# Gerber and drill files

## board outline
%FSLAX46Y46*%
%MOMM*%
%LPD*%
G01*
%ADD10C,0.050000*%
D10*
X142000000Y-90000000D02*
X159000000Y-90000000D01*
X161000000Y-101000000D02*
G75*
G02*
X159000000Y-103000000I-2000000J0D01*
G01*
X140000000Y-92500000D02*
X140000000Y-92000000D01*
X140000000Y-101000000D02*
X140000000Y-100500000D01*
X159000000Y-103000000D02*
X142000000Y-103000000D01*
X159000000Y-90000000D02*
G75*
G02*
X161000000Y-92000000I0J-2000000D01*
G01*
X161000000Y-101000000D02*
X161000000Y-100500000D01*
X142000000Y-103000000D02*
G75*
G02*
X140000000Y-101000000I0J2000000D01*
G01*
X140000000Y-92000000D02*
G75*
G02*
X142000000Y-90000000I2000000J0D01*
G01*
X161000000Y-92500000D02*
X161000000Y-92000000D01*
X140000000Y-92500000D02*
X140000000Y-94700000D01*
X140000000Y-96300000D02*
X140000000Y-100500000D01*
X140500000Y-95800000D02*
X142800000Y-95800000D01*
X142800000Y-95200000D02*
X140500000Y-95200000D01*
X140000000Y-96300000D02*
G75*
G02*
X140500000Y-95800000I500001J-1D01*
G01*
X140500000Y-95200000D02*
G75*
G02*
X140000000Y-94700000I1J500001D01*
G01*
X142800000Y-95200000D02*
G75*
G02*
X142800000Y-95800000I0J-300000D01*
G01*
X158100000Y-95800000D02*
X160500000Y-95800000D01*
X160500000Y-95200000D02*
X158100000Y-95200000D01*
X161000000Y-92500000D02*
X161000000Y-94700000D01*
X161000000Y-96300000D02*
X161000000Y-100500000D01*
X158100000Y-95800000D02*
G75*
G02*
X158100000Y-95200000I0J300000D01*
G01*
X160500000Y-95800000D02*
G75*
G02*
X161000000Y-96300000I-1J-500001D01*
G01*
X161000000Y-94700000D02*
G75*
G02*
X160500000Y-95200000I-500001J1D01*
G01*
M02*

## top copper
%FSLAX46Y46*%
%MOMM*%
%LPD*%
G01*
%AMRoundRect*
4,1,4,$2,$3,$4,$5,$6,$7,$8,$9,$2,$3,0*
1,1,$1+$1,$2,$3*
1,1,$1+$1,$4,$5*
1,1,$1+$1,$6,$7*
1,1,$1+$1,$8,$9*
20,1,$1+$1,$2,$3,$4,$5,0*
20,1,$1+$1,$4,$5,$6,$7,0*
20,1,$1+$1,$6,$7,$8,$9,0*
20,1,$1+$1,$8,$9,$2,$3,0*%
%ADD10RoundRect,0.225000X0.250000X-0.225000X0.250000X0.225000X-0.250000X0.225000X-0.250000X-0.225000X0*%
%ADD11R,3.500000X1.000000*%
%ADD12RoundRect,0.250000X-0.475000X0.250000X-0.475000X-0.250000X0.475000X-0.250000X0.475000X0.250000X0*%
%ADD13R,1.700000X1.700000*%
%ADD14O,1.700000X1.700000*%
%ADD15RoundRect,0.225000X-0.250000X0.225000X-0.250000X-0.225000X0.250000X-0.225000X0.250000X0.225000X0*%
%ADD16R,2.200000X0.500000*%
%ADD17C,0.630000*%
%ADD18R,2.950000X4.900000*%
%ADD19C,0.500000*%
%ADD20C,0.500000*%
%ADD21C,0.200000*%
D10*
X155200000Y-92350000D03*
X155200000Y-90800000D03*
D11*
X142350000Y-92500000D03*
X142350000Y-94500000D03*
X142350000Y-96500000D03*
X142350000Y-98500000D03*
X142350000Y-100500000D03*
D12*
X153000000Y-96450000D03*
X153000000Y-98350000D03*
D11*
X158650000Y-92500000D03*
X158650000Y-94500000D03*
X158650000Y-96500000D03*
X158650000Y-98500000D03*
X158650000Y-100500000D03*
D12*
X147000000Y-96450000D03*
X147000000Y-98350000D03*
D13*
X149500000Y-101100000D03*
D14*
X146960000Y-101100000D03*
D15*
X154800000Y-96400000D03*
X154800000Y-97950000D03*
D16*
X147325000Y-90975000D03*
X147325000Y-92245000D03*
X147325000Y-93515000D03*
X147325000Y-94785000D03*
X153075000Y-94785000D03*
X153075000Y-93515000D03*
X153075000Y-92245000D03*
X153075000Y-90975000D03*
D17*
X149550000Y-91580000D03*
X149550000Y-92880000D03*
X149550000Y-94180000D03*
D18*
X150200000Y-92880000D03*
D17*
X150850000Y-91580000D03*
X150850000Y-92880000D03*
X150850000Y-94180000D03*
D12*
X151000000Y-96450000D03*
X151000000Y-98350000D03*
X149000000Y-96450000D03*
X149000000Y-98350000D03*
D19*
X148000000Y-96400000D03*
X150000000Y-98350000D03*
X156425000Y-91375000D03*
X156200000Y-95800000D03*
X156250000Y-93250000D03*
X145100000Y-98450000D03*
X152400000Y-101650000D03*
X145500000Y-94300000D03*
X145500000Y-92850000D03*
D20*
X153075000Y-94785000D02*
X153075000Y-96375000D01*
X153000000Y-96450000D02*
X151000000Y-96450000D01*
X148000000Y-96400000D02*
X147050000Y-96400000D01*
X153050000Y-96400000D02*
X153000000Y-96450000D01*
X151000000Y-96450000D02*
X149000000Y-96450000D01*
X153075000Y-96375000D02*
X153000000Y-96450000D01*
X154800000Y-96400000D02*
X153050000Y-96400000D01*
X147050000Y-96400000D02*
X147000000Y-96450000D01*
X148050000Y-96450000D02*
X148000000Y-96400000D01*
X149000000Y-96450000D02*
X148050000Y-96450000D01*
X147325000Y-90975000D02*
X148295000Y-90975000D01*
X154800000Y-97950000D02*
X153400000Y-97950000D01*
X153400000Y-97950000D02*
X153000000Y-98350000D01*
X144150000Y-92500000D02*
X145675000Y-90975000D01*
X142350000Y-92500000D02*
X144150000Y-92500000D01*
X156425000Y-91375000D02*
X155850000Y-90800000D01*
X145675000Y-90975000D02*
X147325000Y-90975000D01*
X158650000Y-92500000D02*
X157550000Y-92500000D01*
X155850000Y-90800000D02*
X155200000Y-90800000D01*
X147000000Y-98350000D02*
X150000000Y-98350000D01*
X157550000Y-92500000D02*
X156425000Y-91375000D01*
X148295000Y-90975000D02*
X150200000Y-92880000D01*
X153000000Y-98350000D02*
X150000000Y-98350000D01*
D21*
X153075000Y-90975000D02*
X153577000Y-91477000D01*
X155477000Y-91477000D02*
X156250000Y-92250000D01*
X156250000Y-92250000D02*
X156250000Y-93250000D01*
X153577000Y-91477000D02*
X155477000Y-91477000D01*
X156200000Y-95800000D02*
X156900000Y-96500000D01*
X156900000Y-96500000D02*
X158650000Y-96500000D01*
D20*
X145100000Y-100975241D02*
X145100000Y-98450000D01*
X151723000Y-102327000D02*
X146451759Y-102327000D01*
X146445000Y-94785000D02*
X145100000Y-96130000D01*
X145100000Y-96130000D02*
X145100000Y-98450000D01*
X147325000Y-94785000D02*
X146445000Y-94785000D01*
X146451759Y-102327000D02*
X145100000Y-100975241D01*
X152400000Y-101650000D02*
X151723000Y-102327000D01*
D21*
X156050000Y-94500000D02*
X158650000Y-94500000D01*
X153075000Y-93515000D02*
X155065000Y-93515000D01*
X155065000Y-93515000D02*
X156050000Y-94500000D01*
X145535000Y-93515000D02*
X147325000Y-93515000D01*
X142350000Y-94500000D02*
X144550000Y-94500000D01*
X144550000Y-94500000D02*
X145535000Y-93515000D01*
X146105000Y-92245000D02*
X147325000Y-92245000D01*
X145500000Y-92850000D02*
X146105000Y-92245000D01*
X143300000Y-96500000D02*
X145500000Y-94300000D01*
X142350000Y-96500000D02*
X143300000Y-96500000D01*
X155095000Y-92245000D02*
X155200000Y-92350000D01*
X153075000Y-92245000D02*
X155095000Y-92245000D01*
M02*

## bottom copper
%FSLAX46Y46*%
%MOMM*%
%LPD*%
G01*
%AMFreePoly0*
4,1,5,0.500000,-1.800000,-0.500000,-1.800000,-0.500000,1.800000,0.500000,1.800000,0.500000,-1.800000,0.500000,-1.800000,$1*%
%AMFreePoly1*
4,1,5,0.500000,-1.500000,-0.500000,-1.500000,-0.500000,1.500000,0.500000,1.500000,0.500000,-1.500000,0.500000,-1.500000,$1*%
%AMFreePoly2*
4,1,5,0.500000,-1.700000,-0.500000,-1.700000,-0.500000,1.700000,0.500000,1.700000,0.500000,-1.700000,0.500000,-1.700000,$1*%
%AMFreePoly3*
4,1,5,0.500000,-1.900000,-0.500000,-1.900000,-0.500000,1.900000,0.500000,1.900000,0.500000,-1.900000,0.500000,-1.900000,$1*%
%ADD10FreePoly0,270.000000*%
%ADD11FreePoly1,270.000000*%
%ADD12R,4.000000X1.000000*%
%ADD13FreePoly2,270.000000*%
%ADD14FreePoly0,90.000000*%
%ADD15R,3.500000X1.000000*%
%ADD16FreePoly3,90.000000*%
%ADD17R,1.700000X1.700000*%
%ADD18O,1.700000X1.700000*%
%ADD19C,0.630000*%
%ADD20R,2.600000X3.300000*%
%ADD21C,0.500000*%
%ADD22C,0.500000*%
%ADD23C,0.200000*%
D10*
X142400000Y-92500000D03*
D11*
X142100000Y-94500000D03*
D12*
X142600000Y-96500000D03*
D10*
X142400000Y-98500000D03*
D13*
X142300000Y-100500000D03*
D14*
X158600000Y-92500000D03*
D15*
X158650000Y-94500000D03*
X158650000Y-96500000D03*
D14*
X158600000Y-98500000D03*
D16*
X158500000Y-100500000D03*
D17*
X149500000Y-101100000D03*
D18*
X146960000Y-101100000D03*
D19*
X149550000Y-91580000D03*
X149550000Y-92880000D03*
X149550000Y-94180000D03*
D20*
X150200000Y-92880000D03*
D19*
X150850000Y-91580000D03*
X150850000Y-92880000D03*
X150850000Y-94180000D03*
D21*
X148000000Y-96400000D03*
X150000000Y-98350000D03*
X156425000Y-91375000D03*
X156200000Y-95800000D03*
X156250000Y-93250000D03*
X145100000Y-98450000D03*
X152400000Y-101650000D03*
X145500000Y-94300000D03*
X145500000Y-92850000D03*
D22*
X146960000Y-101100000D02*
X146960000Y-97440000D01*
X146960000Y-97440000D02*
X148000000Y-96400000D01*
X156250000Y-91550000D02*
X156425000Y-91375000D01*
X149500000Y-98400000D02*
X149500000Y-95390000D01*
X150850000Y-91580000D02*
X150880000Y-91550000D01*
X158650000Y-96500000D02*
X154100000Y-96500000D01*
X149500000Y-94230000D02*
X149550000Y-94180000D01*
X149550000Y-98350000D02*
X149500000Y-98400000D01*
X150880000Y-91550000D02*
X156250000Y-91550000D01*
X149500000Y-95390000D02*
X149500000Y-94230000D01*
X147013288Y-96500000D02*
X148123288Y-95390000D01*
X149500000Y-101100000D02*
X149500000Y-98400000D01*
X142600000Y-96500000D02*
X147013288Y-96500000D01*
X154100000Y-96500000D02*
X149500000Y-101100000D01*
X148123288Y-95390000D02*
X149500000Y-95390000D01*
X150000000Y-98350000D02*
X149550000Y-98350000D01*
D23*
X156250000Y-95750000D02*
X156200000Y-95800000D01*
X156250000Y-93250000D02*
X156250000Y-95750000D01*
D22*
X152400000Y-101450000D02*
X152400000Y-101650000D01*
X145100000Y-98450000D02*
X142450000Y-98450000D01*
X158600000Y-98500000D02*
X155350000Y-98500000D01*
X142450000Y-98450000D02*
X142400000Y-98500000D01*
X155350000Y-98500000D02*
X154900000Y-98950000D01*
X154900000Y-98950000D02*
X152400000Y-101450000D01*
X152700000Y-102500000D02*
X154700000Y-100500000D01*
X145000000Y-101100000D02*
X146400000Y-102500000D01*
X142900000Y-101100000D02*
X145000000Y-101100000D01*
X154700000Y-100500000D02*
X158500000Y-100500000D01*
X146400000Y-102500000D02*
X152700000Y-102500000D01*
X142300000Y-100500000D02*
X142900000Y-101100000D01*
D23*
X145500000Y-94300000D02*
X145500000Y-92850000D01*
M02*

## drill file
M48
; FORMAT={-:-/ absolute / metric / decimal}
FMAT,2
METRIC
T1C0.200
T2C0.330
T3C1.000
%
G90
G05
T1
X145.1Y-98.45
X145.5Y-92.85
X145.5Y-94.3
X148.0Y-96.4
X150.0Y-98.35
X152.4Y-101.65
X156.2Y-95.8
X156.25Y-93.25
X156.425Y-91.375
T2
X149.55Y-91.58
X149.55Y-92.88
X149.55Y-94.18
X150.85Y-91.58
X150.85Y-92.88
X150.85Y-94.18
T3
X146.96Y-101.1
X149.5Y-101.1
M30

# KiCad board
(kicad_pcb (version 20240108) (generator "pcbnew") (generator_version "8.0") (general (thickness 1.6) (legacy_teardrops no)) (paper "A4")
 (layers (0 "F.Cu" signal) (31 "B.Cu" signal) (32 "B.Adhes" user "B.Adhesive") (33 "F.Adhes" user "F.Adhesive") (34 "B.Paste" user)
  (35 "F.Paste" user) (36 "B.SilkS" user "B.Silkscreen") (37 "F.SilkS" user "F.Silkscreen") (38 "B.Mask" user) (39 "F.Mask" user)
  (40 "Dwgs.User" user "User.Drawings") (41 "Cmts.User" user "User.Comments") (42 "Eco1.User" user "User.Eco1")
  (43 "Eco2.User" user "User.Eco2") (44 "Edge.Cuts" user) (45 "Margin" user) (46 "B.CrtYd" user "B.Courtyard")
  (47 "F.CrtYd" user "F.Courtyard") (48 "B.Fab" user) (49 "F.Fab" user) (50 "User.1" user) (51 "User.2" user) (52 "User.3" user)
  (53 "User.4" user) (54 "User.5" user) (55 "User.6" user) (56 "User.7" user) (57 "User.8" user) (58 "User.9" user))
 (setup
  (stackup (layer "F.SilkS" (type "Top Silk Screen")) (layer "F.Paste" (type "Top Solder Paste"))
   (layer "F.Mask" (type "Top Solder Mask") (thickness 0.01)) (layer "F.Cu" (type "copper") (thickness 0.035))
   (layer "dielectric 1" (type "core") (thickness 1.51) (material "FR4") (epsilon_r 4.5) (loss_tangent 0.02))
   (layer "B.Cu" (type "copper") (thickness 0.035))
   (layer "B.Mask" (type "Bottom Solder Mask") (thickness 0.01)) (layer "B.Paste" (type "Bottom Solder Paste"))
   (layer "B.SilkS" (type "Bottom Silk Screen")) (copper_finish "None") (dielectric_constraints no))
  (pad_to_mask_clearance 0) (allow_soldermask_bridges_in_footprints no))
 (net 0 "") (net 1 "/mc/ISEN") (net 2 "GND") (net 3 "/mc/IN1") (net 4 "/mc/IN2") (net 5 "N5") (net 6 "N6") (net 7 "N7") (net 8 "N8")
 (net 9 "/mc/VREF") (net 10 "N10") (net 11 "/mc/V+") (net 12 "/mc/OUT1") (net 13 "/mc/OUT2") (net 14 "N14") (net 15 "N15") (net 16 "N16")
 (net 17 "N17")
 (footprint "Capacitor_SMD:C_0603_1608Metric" (layer "F.Cu") (at 155.2 91.575 90)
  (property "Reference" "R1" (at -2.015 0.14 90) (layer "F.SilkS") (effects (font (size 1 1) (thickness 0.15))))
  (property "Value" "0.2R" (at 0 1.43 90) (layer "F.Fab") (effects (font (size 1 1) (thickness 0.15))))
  (pad "1" smd roundrect (at -0.775 0 90) (size 0.9 0.95) (layers "F.Cu" "F.Paste" "F.Mask") (roundrect_rratio 0.25) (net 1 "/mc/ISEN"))
  (pad "2" smd roundrect (at 0.775 0 90) (size 0.9 0.95) (layers "F.Cu" "F.Paste" "F.Mask") (roundrect_rratio 0.25) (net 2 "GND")))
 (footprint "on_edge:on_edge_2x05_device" (layer "F.Cu") (at 140 96.5 -90)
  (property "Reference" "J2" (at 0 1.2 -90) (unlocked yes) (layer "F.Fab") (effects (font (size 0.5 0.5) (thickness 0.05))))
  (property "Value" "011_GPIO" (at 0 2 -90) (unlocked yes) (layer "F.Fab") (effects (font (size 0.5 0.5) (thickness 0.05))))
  (fp_line (start -4 0) (end -1.8 0) (stroke (width 0.05) (type solid)) (layer "Edge.Cuts"))
  (fp_line (start -0.2 0) (end 4 0) (stroke (width 0.05) (type solid)) (layer "Edge.Cuts"))
  (fp_line (start -0.7 -0.5) (end -0.7 -2.8) (stroke (width 0.05) (type solid)) (layer "Edge.Cuts"))
  (fp_line (start -1.3 -2.8) (end -1.3 -0.5) (stroke (width 0.05) (type solid)) (layer "Edge.Cuts"))
  (fp_arc (start -0.2 0) (mid -0.553553 -0.146447) (end -0.7 -0.5) (stroke (width 0.05) (type solid)) (layer "Edge.Cuts"))
  (fp_arc (start -1.3 -0.5) (mid -1.446447 -0.146447) (end -1.8 0) (stroke (width 0.05) (type solid)) (layer "Edge.Cuts"))
  (fp_arc (start -1.3 -2.8) (mid -1 -3.1) (end -0.7 -2.8) (stroke (width 0.05) (type solid)) (layer "Edge.Cuts"))
  (pad "1" smd rect (at -4 -2.35 90) (size 1 3.5) (layers "F.Cu" "F.Mask") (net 2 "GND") (zone_connect 0))
  (pad "2" smd rect (at -2 -2.35 270) (size 1 3.5) (layers "F.Cu" "F.Mask") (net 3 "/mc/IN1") (zone_connect 0))
  (pad "3" smd rect (at 0 -2.35 270) (size 1 3.5) (layers "F.Cu" "F.Mask") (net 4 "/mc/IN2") (zone_connect 0))
  (pad "4" smd rect (at 2 -2.35 90) (size 1 3.5) (layers "F.Cu" "F.Mask") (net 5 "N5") (zone_connect 0))
  (pad "5" smd rect (at 4 -2.35 90) (size 1 3.5) (layers "F.Cu" "F.Mask") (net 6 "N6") (zone_connect 0))
  (pad "6" smd custom (at -4 -2.4 270) (size 1 3.6) (layers "B.Cu" "B.Mask") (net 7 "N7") (zone_connect 0)
   (options (clearance outline) (anchor rect)) (primitives))
  (pad "7" smd custom (at -2 -2.1 270) (size 1 3) (layers "B.Cu" "B.Mask") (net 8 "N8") (zone_connect 0)
   (options (clearance outline) (anchor rect)) (primitives))
  (pad "8" smd rect (at 0 -2.6 270) (size 1 4) (layers "B.Cu" "B.Mask") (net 2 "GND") (zone_connect 0))
  (pad "9" smd custom (at 2 -2.4 270) (size 1 3.6) (layers "B.Cu" "B.Mask") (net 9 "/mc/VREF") (zone_connect 0)
   (options (clearance outline) (anchor rect)) (primitives))
  (pad "10" smd custom (at 4 -2.3 270) (size 1 3.4) (layers "B.Cu" "B.Mask") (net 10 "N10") (zone_connect 0)
   (options (clearance outline) (anchor rect)) (primitives))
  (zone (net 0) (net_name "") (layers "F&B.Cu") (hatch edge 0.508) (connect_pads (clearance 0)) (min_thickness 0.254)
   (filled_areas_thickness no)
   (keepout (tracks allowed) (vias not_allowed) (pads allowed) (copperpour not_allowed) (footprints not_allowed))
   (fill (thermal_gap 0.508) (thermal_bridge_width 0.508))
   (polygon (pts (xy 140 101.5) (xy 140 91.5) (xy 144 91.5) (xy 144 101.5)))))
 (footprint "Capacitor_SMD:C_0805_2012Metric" (layer "F.Cu") (at 153 97.4 -90)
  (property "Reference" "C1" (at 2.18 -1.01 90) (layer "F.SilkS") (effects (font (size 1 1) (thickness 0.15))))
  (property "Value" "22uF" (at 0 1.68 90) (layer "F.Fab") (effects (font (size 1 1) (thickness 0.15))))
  (pad "1" smd roundrect (at -0.95 0 270) (size 1 1.45) (layers "F.Cu" "F.Paste" "F.Mask") (roundrect_rratio 0.25) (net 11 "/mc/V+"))
  (pad "2" smd roundrect (at 0.95 0 270) (size 1 1.45) (layers "F.Cu" "F.Paste" "F.Mask") (roundrect_rratio 0.25) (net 2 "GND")))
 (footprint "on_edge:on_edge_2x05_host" (layer "F.Cu") (at 161 96.5 -90)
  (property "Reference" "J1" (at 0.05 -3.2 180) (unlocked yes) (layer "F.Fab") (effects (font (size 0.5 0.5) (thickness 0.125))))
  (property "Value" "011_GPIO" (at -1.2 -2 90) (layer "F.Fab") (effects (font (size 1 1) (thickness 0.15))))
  (fp_line (start -0.7 2.9) (end -0.7 0.5) (stroke (width 0.05) (type solid)) (layer "Edge.Cuts"))
  (fp_line (start -1.3 0.5) (end -1.3 2.9) (stroke (width 0.05) (type solid)) (layer "Edge.Cuts"))
  (fp_line (start -4 0) (end -1.8 0) (stroke (width 0.05) (type solid)) (layer "Edge.Cuts"))
  (fp_line (start -0.2 0) (end 4 0) (stroke (width 0.05) (type solid)) (layer "Edge.Cuts"))
  (fp_arc (start -0.7 2.9) (mid -1 3.2) (end -1.3 2.9) (stroke (width 0.05) (type solid)) (layer "Edge.Cuts"))
  (fp_arc (start -0.7 0.5) (mid -0.553553 0.146447) (end -0.2 0) (stroke (width 0.05) (type solid)) (layer "Edge.Cuts"))
  (fp_arc (start -1.8 0) (mid -1.446447 0.146447) (end -1.3 0.5) (stroke (width 0.05) (type solid)) (layer "Edge.Cuts"))
  (pad "1" smd rect (at -4 2.35 270) (size 1 3.5) (layers "F.Cu" "F.Mask") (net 2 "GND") (zone_connect 0))
  (pad "2" smd rect (at -2 2.35 270) (size 1 3.5) (layers "F.Cu" "F.Mask") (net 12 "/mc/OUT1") (zone_connect 0))
  (pad "3" smd rect (at 0 2.35 270) (size 1 3.5) (layers "F.Cu" "F.Mask") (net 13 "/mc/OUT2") (zone_connect 0))
  (pad "4" smd rect (at 2 2.35 270) (size 1 3.5) (layers "F.Cu" "F.Mask") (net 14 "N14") (zone_connect 0))
  (pad "5" smd rect (at 4 2.35 270) (size 1 3.5) (layers "F.Cu" "F.Mask") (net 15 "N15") (zone_connect 0))
  (pad "6" smd custom (at -4 2.4 90) (size 1 3.6) (layers "B.Cu" "B.Mask") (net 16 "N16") (zone_connect 0)
   (options (clearance outline) (anchor rect)) (primitives))
  (pad "7" smd rect (at -2 2.35 90) (size 1 3.5) (layers "B.Cu" "B.Mask") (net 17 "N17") (zone_connect 0))
  (pad "8" smd rect (at 0 2.35 90) (size 1 3.5) (layers "B.Cu" "B.Mask") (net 2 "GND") (zone_connect 0))
  (pad "9" smd custom (at 2 2.4 90) (size 1 3.6) (layers "B.Cu" "B.Mask") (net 9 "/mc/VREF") (zone_connect 0)
   (options (clearance outline) (anchor rect)) (primitives))
  (pad "10" smd custom (at 4 2.5 90) (size 1 3.8) (layers "B.Cu" "B.Mask") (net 10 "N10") (zone_connect 0)
   (options (clearance outline) (anchor rect)) (primitives))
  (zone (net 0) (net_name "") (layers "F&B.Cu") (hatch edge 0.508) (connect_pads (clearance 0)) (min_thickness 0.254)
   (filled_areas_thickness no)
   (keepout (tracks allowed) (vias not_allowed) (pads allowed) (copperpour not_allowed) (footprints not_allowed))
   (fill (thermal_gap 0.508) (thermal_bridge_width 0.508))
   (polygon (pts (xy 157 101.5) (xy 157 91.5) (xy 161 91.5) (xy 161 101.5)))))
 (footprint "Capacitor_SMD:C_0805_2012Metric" (layer "F.Cu") (at 147 97.4 -90)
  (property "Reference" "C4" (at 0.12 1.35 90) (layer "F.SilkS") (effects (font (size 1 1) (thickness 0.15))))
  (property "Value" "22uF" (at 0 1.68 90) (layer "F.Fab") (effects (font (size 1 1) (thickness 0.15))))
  (pad "1" smd roundrect (at -0.95 0 270) (size 1 1.45) (layers "F.Cu" "F.Paste" "F.Mask") (roundrect_rratio 0.25) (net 11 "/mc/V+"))
  (pad "2" smd roundrect (at 0.95 0 270) (size 1 1.45) (layers "F.Cu" "F.Paste" "F.Mask") (roundrect_rratio 0.25) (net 2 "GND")))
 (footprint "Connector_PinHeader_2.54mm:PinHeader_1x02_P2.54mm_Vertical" (layer "F.Cu") (at 149.5 101.1 -90)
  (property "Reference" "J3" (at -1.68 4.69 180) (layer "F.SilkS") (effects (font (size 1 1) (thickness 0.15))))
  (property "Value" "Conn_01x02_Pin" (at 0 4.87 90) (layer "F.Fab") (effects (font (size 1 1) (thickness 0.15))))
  (pad "1" thru_hole rect (at 0 0 270) (size 1.7 1.7) (drill 1) (layers "*.Cu" "*.Mask") (remove_unused_layers no) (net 2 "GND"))
  (pad "2" thru_hole oval (at 0 2.54 270) (size 1.7 1.7) (drill 1) (layers "*.Cu" "*.Mask") (remove_unused_layers no) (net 11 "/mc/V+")))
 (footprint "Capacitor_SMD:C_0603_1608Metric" (layer "F.Cu") (at 154.8 97.175 -90)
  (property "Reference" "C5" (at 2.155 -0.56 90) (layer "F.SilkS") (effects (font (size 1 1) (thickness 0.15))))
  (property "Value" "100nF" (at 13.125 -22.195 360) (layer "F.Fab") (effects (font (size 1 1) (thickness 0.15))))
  (pad "1" smd roundrect (at -0.775 0 270) (size 0.9 0.95) (layers "F.Cu" "F.Paste" "F.Mask") (roundrect_rratio 0.25) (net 11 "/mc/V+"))
  (pad "2" smd roundrect (at 0.775 0 270) (size 0.9 0.95) (layers "F.Cu" "F.Paste" "F.Mask") (roundrect_rratio 0.25) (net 2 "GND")))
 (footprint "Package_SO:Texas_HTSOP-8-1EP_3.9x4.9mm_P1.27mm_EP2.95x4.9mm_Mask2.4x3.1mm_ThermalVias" (layer "F.Cu") (at 150.2 92.88)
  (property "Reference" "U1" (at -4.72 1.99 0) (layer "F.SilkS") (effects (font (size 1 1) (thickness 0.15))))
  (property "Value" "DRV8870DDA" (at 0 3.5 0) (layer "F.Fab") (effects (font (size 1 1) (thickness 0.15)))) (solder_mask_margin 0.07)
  (pad "" smd rect (at 0 0) (size 2.4 3.1) (layers "F.Paste")) (pad "" smd rect (at 0 0) (size 2.4 3.1) (layers "F.Mask"))
  (pad "1" smd rect (at -2.875 -1.905) (size 2.2 0.5) (layers "F.Cu" "F.Paste" "F.Mask") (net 2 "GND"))
  (pad "2" smd rect (at -2.875 -0.635) (size 2.2 0.5) (layers "F.Cu" "F.Paste" "F.Mask") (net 4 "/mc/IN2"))
  (pad "3" smd rect (at -2.875 0.635) (size 2.2 0.5) (layers "F.Cu" "F.Paste" "F.Mask") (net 3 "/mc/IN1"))
  (pad "4" smd rect (at -2.875 1.905) (size 2.2 0.5) (layers "F.Cu" "F.Paste" "F.Mask") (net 9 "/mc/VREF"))
  (pad "5" smd rect (at 2.875 1.905) (size 2.2 0.5) (layers "F.Cu" "F.Paste" "F.Mask") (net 11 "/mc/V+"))
  (pad "6" smd rect (at 2.875 0.635) (size 2.2 0.5) (layers "F.Cu" "F.Paste" "F.Mask") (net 12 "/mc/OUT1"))
  (pad "7" smd rect (at 2.875 -0.635) (size 2.2 0.5) (layers "F.Cu" "F.Paste" "F.Mask") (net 1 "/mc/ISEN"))
  (pad "8" smd rect (at 2.875 -1.905) (size 2.2 0.5) (layers "F.Cu" "F.Paste" "F.Mask") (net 13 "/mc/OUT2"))
  (pad "9" thru_hole circle (at -0.65 -1.3) (size 0.63 0.63) (drill 0.33) (layers "*.Cu" "*.Mask") (remove_unused_layers no) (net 2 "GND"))
  (pad "9" thru_hole circle (at -0.65 0) (size 0.63 0.63) (drill 0.33) (layers "*.Cu" "*.Mask") (remove_unused_layers no) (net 2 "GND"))
  (pad "9" thru_hole circle (at -0.65 1.3) (size 0.63 0.63) (drill 0.33) (layers "*.Cu" "*.Mask") (remove_unused_layers no) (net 2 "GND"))
  (pad "9" smd rect (at 0 0) (size 2.6 3.3) (layers "B.Cu") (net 2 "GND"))
  (pad "9" smd rect (at 0 0) (size 2.95 4.9) (layers "F.Cu") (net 2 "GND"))
  (pad "9" thru_hole circle (at 0.65 -1.3) (size 0.63 0.63) (drill 0.33) (layers "*.Cu" "*.Mask") (remove_unused_layers no) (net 2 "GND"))
  (pad "9" thru_hole circle (at 0.65 0) (size 0.63 0.63) (drill 0.33) (layers "*.Cu" "*.Mask") (remove_unused_layers no) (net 2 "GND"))
  (pad "9" thru_hole circle (at 0.65 1.3) (size 0.63 0.63) (drill 0.33) (layers "*.Cu" "*.Mask") (remove_unused_layers no) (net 2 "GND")))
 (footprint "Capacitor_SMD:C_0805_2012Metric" (layer "F.Cu") (at 151 97.4 -90)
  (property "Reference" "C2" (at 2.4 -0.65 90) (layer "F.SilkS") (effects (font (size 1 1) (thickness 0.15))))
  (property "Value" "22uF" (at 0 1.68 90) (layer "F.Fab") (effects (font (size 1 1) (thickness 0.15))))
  (pad "1" smd roundrect (at -0.95 0 270) (size 1 1.45) (layers "F.Cu" "F.Paste" "F.Mask") (roundrect_rratio 0.25) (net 11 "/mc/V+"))
  (pad "2" smd roundrect (at 0.95 0 270) (size 1 1.45) (layers "F.Cu" "F.Paste" "F.Mask") (roundrect_rratio 0.25) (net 2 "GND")))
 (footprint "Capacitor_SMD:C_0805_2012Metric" (layer "F.Cu") (at 149 97.4 -90)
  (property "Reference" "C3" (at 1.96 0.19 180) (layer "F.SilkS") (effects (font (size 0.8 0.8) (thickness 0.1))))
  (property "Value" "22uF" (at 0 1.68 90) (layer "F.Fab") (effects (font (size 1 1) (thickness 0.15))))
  (pad "1" smd roundrect (at -0.95 0 270) (size 1 1.45) (layers "F.Cu" "F.Paste" "F.Mask") (roundrect_rratio 0.25) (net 11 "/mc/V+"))
  (pad "2" smd roundrect (at 0.95 0 270) (size 1 1.45) (layers "F.Cu" "F.Paste" "F.Mask") (roundrect_rratio 0.25) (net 2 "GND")))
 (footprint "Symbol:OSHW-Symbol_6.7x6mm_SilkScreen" (layer "B.Cu") (at 150.12 97.58 180)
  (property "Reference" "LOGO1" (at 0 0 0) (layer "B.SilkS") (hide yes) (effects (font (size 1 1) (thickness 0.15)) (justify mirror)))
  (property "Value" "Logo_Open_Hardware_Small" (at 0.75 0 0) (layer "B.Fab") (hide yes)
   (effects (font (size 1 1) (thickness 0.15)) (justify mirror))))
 (gr_line (start 142 90) (end 159 90) (stroke (width 0.05) (type solid)) (layer "Edge.Cuts"))
 (gr_arc (start 161 101) (mid 160.414214 102.414214) (end 159 103) (stroke (width 0.05) (type solid)) (layer "Edge.Cuts"))
 (gr_line (start 140 92.5) (end 140 92) (stroke (width 0.05) (type default)) (layer "Edge.Cuts"))
 (gr_line (start 140 101) (end 140 100.5) (stroke (width 0.05) (type default)) (layer "Edge.Cuts"))
 (gr_line (start 159 103) (end 142 103) (stroke (width 0.05) (type solid)) (layer "Edge.Cuts"))
 (gr_arc (start 159 90) (mid 160.414214 90.585786) (end 161 92) (stroke (width 0.05) (type solid)) (layer "Edge.Cuts"))
 (gr_line (start 161 101) (end 161 100.5) (stroke (width 0.05) (type default)) (layer "Edge.Cuts"))
 (gr_arc (start 142 103) (mid 140.585786 102.414214) (end 140 101) (stroke (width 0.05) (type solid)) (layer "Edge.Cuts"))
 (gr_arc (start 140 92) (mid 140.585786 90.585786) (end 142 90) (stroke (width 0.05) (type solid)) (layer "Edge.Cuts"))
 (gr_line (start 161 92.5) (end 161 92) (stroke (width 0.05) (type default)) (layer "Edge.Cuts"))
 (segment (start 153.075 94.785) (end 153.075 96.375) (width 0.5) (layer "F.Cu") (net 11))
 (segment (start 153 96.45) (end 151 96.45) (width 0.5) (layer "F.Cu") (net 11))
 (segment (start 148 96.4) (end 147.05 96.4) (width 0.5) (layer "F.Cu") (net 11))
 (segment (start 153.05 96.4) (end 153 96.45) (width 0.5) (layer "F.Cu") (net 11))
 (segment (start 151 96.45) (end 149 96.45) (width 0.5) (layer "F.Cu") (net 11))
 (segment (start 153.075 96.375) (end 153 96.45) (width 0.5) (layer "F.Cu") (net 11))
 (segment (start 154.8 96.4) (end 153.05 96.4) (width 0.5) (layer "F.Cu") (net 11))
 (segment (start 147.05 96.4) (end 147 96.45) (width 0.5) (layer "F.Cu") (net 11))
 (segment (start 148.05 96.45) (end 148 96.4) (width 0.5) (layer "F.Cu") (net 11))
 (segment (start 149 96.45) (end 148.05 96.45) (width 0.5) (layer "F.Cu") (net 11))
 (via (at 148 96.4) (size 0.5) (drill 0.2) (layers "F.Cu" "B.Cu") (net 11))
 (segment (start 146.96 101.1) (end 146.96 97.44) (width 0.5) (layer "B.Cu") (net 11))
 (segment (start 146.96 97.44) (end 148 96.4) (width 0.5) (layer "B.Cu") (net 11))
 (segment (start 147.325 90.975) (end 148.295 90.975) (width 0.5) (layer "F.Cu") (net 2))
 (segment (start 154.8 97.95) (end 153.4 97.95) (width 0.5) (layer "F.Cu") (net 2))
 (segment (start 153.4 97.95) (end 153 98.35) (width 0.5) (layer "F.Cu") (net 2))
 (segment (start 144.15 92.5) (end 145.675 90.975) (width 0.5) (layer "F.Cu") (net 2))
 (segment (start 142.35 92.5) (end 144.15 92.5) (width 0.5) (layer "F.Cu") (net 2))
 (segment (start 156.425 91.375) (end 155.85 90.8) (width 0.5) (layer "F.Cu") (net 2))
 (segment (start 145.675 90.975) (end 147.325 90.975) (width 0.5) (layer "F.Cu") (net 2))
 (segment (start 158.65 92.5) (end 157.55 92.5) (width 0.5) (layer "F.Cu") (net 2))
 (segment (start 155.85 90.8) (end 155.2 90.8) (width 0.5) (layer "F.Cu") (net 2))
 (segment (start 147 98.35) (end 150 98.35) (width 0.5) (layer "F.Cu") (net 2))
 (segment (start 157.55 92.5) (end 156.425 91.375) (width 0.5) (layer "F.Cu") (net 2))
 (segment (start 148.295 90.975) (end 150.2 92.88) (width 0.5) (layer "F.Cu") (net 2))
 (segment (start 153 98.35) (end 150 98.35) (width 0.5) (layer "F.Cu") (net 2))
 (via (at 150 98.35) (size 0.5) (drill 0.2) (layers "F.Cu" "B.Cu") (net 2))
 (via (at 156.425 91.375) (size 0.5) (drill 0.2) (layers "F.Cu" "B.Cu") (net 2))
 (segment (start 156.25 91.55) (end 156.425 91.375) (width 0.5) (layer "B.Cu") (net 2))
 (segment (start 149.5 98.4) (end 149.5 95.39) (width 0.5) (layer "B.Cu") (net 2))
 (segment (start 150.85 91.58) (end 150.88 91.55) (width 0.5) (layer "B.Cu") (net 2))
 (segment (start 158.65 96.5) (end 154.1 96.5) (width 0.5) (layer "B.Cu") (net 2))
 (segment (start 149.5 94.23) (end 149.55 94.18) (width 0.5) (layer "B.Cu") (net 2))
 (segment (start 149.55 98.35) (end 149.5 98.4) (width 0.5) (layer "B.Cu") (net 2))
 (segment (start 150.88 91.55) (end 156.25 91.55) (width 0.5) (layer "B.Cu") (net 2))
 (segment (start 149.5 95.39) (end 149.5 94.23) (width 0.5) (layer "B.Cu") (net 2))
 (segment (start 147.013288 96.5) (end 148.123288 95.39) (width 0.5) (layer "B.Cu") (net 2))
 (segment (start 149.5 101.1) (end 149.5 98.4) (width 0.5) (layer "B.Cu") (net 2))
 (segment (start 142.6 96.5) (end 147.013288 96.5) (width 0.5) (layer "B.Cu") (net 2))
 (segment (start 154.1 96.5) (end 149.5 101.1) (width 0.5) (layer "B.Cu") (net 2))
 (segment (start 148.123288 95.39) (end 149.5 95.39) (width 0.5) (layer "B.Cu") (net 2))
 (segment (start 150 98.35) (end 149.55 98.35) (width 0.5) (layer "B.Cu") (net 2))
 (segment (start 153.075 90.975) (end 153.577 91.477) (width 0.2) (layer "F.Cu") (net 13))
 (segment (start 155.477 91.477) (end 156.25 92.25) (width 0.2) (layer "F.Cu") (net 13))
 (segment (start 156.25 92.25) (end 156.25 93.25) (width 0.2) (layer "F.Cu") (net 13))
 (segment (start 153.577 91.477) (end 155.477 91.477) (width 0.2) (layer "F.Cu") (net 13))
 (segment (start 156.2 95.8) (end 156.9 96.5) (width 0.2) (layer "F.Cu") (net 13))
 (segment (start 156.9 96.5) (end 158.65 96.5) (width 0.2) (layer "F.Cu") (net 13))
 (via (at 156.2 95.8) (size 0.5) (drill 0.2) (layers "F.Cu" "B.Cu") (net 13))
 (via (at 156.25 93.25) (size 0.5) (drill 0.2) (layers "F.Cu" "B.Cu") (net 13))
 (segment (start 156.25 95.75) (end 156.2 95.8) (width 0.2) (layer "B.Cu") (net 13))
 (segment (start 156.25 93.25) (end 156.25 95.75) (width 0.2) (layer "B.Cu") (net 13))
 (segment (start 145.1 100.975241) (end 145.1 98.45) (width 0.5) (layer "F.Cu") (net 9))
 (segment (start 151.723 102.327) (end 146.451759 102.327) (width 0.5) (layer "F.Cu") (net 9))
 (segment (start 146.445 94.785) (end 145.1 96.13) (width 0.5) (layer "F.Cu") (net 9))
 (segment (start 145.1 96.13) (end 145.1 98.45) (width 0.5) (layer "F.Cu") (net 9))
 (segment (start 147.325 94.785) (end 146.445 94.785) (width 0.5) (layer "F.Cu") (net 9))
 (segment (start 146.451759 102.327) (end 145.1 100.975241) (width 0.5) (layer "F.Cu") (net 9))
 (segment (start 152.4 101.65) (end 151.723 102.327) (width 0.5) (layer "F.Cu") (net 9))
 (via (at 145.1 98.45) (size 0.5) (drill 0.2) (layers "F.Cu" "B.Cu") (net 9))
 (via (at 152.4 101.65) (size 0.5) (drill 0.2) (layers "F.Cu" "B.Cu") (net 9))
 (segment (start 152.4 101.45) (end 152.4 101.65) (width 0.5) (layer "B.Cu") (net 9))
 (segment (start 145.1 98.45) (end 142.45 98.45) (width 0.5) (layer "B.Cu") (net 9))
 (segment (start 158.6 98.5) (end 155.35 98.5) (width 0.5) (layer "B.Cu") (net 9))
 (segment (start 142.45 98.45) (end 142.4 98.5) (width 0.5) (layer "B.Cu") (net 9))
 (segment (start 155.35 98.5) (end 154.9 98.95) (width 0.5) (layer "B.Cu") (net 9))
 (segment (start 154.9 98.95) (end 152.4 101.45) (width 0.5) (layer "B.Cu") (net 9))
 (segment (start 156.05 94.5) (end 158.65 94.5) (width 0.2) (layer "F.Cu") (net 12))
 (segment (start 153.075 93.515) (end 155.065 93.515) (width 0.2) (layer "F.Cu") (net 12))
 (segment (start 155.065 93.515) (end 156.05 94.5) (width 0.2) (layer "F.Cu") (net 12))
 (segment (start 152.7 102.5) (end 154.7 100.5) (width 0.5) (layer "B.Cu") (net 10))
 (segment (start 145 101.1) (end 146.4 102.5) (width 0.5) (layer "B.Cu") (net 10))
 (segment (start 142.9 101.1) (end 145 101.1) (width 0.5) (layer "B.Cu") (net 10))
 (segment (start 154.7 100.5) (end 158.5 100.5) (width 0.5) (layer "B.Cu") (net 10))
 (segment (start 146.4 102.5) (end 152.7 102.5) (width 0.5) (layer "B.Cu") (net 10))
 (segment (start 142.3 100.5) (end 142.9 101.1) (width 0.5) (layer "B.Cu") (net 10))
 (segment (start 145.535 93.515) (end 147.325 93.515) (width 0.2) (layer "F.Cu") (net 3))
 (segment (start 142.35 94.5) (end 144.55 94.5) (width 0.2) (layer "F.Cu") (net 3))
 (segment (start 144.55 94.5) (end 145.535 93.515) (width 0.2) (layer "F.Cu") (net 3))
 (segment (start 146.105 92.245) (end 147.325 92.245) (width 0.2) (layer "F.Cu") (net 4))
 (segment (start 145.5 92.85) (end 146.105 92.245) (width 0.2) (layer "F.Cu") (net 4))
 (segment (start 143.3 96.5) (end 145.5 94.3) (width 0.2) (layer "F.Cu") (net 4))
 (segment (start 142.35 96.5) (end 143.3 96.5) (width 0.2) (layer "F.Cu") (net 4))
 (via (at 145.5 94.3) (size 0.5) (drill 0.2) (layers "F.Cu" "B.Cu") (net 4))
 (via (at 145.5 92.85) (size 0.5) (drill 0.2) (layers "F.Cu" "B.Cu") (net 4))
 (segment (start 145.5 94.3) (end 145.5 92.85) (width 0.2) (layer "B.Cu") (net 4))
 (segment (start 155.095 92.245) (end 155.2 92.35) (width 0.2) (layer "F.Cu") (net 1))
 (segment (start 153.075 92.245) (end 155.095 92.245) (width 0.2) (layer "F.Cu") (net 1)))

